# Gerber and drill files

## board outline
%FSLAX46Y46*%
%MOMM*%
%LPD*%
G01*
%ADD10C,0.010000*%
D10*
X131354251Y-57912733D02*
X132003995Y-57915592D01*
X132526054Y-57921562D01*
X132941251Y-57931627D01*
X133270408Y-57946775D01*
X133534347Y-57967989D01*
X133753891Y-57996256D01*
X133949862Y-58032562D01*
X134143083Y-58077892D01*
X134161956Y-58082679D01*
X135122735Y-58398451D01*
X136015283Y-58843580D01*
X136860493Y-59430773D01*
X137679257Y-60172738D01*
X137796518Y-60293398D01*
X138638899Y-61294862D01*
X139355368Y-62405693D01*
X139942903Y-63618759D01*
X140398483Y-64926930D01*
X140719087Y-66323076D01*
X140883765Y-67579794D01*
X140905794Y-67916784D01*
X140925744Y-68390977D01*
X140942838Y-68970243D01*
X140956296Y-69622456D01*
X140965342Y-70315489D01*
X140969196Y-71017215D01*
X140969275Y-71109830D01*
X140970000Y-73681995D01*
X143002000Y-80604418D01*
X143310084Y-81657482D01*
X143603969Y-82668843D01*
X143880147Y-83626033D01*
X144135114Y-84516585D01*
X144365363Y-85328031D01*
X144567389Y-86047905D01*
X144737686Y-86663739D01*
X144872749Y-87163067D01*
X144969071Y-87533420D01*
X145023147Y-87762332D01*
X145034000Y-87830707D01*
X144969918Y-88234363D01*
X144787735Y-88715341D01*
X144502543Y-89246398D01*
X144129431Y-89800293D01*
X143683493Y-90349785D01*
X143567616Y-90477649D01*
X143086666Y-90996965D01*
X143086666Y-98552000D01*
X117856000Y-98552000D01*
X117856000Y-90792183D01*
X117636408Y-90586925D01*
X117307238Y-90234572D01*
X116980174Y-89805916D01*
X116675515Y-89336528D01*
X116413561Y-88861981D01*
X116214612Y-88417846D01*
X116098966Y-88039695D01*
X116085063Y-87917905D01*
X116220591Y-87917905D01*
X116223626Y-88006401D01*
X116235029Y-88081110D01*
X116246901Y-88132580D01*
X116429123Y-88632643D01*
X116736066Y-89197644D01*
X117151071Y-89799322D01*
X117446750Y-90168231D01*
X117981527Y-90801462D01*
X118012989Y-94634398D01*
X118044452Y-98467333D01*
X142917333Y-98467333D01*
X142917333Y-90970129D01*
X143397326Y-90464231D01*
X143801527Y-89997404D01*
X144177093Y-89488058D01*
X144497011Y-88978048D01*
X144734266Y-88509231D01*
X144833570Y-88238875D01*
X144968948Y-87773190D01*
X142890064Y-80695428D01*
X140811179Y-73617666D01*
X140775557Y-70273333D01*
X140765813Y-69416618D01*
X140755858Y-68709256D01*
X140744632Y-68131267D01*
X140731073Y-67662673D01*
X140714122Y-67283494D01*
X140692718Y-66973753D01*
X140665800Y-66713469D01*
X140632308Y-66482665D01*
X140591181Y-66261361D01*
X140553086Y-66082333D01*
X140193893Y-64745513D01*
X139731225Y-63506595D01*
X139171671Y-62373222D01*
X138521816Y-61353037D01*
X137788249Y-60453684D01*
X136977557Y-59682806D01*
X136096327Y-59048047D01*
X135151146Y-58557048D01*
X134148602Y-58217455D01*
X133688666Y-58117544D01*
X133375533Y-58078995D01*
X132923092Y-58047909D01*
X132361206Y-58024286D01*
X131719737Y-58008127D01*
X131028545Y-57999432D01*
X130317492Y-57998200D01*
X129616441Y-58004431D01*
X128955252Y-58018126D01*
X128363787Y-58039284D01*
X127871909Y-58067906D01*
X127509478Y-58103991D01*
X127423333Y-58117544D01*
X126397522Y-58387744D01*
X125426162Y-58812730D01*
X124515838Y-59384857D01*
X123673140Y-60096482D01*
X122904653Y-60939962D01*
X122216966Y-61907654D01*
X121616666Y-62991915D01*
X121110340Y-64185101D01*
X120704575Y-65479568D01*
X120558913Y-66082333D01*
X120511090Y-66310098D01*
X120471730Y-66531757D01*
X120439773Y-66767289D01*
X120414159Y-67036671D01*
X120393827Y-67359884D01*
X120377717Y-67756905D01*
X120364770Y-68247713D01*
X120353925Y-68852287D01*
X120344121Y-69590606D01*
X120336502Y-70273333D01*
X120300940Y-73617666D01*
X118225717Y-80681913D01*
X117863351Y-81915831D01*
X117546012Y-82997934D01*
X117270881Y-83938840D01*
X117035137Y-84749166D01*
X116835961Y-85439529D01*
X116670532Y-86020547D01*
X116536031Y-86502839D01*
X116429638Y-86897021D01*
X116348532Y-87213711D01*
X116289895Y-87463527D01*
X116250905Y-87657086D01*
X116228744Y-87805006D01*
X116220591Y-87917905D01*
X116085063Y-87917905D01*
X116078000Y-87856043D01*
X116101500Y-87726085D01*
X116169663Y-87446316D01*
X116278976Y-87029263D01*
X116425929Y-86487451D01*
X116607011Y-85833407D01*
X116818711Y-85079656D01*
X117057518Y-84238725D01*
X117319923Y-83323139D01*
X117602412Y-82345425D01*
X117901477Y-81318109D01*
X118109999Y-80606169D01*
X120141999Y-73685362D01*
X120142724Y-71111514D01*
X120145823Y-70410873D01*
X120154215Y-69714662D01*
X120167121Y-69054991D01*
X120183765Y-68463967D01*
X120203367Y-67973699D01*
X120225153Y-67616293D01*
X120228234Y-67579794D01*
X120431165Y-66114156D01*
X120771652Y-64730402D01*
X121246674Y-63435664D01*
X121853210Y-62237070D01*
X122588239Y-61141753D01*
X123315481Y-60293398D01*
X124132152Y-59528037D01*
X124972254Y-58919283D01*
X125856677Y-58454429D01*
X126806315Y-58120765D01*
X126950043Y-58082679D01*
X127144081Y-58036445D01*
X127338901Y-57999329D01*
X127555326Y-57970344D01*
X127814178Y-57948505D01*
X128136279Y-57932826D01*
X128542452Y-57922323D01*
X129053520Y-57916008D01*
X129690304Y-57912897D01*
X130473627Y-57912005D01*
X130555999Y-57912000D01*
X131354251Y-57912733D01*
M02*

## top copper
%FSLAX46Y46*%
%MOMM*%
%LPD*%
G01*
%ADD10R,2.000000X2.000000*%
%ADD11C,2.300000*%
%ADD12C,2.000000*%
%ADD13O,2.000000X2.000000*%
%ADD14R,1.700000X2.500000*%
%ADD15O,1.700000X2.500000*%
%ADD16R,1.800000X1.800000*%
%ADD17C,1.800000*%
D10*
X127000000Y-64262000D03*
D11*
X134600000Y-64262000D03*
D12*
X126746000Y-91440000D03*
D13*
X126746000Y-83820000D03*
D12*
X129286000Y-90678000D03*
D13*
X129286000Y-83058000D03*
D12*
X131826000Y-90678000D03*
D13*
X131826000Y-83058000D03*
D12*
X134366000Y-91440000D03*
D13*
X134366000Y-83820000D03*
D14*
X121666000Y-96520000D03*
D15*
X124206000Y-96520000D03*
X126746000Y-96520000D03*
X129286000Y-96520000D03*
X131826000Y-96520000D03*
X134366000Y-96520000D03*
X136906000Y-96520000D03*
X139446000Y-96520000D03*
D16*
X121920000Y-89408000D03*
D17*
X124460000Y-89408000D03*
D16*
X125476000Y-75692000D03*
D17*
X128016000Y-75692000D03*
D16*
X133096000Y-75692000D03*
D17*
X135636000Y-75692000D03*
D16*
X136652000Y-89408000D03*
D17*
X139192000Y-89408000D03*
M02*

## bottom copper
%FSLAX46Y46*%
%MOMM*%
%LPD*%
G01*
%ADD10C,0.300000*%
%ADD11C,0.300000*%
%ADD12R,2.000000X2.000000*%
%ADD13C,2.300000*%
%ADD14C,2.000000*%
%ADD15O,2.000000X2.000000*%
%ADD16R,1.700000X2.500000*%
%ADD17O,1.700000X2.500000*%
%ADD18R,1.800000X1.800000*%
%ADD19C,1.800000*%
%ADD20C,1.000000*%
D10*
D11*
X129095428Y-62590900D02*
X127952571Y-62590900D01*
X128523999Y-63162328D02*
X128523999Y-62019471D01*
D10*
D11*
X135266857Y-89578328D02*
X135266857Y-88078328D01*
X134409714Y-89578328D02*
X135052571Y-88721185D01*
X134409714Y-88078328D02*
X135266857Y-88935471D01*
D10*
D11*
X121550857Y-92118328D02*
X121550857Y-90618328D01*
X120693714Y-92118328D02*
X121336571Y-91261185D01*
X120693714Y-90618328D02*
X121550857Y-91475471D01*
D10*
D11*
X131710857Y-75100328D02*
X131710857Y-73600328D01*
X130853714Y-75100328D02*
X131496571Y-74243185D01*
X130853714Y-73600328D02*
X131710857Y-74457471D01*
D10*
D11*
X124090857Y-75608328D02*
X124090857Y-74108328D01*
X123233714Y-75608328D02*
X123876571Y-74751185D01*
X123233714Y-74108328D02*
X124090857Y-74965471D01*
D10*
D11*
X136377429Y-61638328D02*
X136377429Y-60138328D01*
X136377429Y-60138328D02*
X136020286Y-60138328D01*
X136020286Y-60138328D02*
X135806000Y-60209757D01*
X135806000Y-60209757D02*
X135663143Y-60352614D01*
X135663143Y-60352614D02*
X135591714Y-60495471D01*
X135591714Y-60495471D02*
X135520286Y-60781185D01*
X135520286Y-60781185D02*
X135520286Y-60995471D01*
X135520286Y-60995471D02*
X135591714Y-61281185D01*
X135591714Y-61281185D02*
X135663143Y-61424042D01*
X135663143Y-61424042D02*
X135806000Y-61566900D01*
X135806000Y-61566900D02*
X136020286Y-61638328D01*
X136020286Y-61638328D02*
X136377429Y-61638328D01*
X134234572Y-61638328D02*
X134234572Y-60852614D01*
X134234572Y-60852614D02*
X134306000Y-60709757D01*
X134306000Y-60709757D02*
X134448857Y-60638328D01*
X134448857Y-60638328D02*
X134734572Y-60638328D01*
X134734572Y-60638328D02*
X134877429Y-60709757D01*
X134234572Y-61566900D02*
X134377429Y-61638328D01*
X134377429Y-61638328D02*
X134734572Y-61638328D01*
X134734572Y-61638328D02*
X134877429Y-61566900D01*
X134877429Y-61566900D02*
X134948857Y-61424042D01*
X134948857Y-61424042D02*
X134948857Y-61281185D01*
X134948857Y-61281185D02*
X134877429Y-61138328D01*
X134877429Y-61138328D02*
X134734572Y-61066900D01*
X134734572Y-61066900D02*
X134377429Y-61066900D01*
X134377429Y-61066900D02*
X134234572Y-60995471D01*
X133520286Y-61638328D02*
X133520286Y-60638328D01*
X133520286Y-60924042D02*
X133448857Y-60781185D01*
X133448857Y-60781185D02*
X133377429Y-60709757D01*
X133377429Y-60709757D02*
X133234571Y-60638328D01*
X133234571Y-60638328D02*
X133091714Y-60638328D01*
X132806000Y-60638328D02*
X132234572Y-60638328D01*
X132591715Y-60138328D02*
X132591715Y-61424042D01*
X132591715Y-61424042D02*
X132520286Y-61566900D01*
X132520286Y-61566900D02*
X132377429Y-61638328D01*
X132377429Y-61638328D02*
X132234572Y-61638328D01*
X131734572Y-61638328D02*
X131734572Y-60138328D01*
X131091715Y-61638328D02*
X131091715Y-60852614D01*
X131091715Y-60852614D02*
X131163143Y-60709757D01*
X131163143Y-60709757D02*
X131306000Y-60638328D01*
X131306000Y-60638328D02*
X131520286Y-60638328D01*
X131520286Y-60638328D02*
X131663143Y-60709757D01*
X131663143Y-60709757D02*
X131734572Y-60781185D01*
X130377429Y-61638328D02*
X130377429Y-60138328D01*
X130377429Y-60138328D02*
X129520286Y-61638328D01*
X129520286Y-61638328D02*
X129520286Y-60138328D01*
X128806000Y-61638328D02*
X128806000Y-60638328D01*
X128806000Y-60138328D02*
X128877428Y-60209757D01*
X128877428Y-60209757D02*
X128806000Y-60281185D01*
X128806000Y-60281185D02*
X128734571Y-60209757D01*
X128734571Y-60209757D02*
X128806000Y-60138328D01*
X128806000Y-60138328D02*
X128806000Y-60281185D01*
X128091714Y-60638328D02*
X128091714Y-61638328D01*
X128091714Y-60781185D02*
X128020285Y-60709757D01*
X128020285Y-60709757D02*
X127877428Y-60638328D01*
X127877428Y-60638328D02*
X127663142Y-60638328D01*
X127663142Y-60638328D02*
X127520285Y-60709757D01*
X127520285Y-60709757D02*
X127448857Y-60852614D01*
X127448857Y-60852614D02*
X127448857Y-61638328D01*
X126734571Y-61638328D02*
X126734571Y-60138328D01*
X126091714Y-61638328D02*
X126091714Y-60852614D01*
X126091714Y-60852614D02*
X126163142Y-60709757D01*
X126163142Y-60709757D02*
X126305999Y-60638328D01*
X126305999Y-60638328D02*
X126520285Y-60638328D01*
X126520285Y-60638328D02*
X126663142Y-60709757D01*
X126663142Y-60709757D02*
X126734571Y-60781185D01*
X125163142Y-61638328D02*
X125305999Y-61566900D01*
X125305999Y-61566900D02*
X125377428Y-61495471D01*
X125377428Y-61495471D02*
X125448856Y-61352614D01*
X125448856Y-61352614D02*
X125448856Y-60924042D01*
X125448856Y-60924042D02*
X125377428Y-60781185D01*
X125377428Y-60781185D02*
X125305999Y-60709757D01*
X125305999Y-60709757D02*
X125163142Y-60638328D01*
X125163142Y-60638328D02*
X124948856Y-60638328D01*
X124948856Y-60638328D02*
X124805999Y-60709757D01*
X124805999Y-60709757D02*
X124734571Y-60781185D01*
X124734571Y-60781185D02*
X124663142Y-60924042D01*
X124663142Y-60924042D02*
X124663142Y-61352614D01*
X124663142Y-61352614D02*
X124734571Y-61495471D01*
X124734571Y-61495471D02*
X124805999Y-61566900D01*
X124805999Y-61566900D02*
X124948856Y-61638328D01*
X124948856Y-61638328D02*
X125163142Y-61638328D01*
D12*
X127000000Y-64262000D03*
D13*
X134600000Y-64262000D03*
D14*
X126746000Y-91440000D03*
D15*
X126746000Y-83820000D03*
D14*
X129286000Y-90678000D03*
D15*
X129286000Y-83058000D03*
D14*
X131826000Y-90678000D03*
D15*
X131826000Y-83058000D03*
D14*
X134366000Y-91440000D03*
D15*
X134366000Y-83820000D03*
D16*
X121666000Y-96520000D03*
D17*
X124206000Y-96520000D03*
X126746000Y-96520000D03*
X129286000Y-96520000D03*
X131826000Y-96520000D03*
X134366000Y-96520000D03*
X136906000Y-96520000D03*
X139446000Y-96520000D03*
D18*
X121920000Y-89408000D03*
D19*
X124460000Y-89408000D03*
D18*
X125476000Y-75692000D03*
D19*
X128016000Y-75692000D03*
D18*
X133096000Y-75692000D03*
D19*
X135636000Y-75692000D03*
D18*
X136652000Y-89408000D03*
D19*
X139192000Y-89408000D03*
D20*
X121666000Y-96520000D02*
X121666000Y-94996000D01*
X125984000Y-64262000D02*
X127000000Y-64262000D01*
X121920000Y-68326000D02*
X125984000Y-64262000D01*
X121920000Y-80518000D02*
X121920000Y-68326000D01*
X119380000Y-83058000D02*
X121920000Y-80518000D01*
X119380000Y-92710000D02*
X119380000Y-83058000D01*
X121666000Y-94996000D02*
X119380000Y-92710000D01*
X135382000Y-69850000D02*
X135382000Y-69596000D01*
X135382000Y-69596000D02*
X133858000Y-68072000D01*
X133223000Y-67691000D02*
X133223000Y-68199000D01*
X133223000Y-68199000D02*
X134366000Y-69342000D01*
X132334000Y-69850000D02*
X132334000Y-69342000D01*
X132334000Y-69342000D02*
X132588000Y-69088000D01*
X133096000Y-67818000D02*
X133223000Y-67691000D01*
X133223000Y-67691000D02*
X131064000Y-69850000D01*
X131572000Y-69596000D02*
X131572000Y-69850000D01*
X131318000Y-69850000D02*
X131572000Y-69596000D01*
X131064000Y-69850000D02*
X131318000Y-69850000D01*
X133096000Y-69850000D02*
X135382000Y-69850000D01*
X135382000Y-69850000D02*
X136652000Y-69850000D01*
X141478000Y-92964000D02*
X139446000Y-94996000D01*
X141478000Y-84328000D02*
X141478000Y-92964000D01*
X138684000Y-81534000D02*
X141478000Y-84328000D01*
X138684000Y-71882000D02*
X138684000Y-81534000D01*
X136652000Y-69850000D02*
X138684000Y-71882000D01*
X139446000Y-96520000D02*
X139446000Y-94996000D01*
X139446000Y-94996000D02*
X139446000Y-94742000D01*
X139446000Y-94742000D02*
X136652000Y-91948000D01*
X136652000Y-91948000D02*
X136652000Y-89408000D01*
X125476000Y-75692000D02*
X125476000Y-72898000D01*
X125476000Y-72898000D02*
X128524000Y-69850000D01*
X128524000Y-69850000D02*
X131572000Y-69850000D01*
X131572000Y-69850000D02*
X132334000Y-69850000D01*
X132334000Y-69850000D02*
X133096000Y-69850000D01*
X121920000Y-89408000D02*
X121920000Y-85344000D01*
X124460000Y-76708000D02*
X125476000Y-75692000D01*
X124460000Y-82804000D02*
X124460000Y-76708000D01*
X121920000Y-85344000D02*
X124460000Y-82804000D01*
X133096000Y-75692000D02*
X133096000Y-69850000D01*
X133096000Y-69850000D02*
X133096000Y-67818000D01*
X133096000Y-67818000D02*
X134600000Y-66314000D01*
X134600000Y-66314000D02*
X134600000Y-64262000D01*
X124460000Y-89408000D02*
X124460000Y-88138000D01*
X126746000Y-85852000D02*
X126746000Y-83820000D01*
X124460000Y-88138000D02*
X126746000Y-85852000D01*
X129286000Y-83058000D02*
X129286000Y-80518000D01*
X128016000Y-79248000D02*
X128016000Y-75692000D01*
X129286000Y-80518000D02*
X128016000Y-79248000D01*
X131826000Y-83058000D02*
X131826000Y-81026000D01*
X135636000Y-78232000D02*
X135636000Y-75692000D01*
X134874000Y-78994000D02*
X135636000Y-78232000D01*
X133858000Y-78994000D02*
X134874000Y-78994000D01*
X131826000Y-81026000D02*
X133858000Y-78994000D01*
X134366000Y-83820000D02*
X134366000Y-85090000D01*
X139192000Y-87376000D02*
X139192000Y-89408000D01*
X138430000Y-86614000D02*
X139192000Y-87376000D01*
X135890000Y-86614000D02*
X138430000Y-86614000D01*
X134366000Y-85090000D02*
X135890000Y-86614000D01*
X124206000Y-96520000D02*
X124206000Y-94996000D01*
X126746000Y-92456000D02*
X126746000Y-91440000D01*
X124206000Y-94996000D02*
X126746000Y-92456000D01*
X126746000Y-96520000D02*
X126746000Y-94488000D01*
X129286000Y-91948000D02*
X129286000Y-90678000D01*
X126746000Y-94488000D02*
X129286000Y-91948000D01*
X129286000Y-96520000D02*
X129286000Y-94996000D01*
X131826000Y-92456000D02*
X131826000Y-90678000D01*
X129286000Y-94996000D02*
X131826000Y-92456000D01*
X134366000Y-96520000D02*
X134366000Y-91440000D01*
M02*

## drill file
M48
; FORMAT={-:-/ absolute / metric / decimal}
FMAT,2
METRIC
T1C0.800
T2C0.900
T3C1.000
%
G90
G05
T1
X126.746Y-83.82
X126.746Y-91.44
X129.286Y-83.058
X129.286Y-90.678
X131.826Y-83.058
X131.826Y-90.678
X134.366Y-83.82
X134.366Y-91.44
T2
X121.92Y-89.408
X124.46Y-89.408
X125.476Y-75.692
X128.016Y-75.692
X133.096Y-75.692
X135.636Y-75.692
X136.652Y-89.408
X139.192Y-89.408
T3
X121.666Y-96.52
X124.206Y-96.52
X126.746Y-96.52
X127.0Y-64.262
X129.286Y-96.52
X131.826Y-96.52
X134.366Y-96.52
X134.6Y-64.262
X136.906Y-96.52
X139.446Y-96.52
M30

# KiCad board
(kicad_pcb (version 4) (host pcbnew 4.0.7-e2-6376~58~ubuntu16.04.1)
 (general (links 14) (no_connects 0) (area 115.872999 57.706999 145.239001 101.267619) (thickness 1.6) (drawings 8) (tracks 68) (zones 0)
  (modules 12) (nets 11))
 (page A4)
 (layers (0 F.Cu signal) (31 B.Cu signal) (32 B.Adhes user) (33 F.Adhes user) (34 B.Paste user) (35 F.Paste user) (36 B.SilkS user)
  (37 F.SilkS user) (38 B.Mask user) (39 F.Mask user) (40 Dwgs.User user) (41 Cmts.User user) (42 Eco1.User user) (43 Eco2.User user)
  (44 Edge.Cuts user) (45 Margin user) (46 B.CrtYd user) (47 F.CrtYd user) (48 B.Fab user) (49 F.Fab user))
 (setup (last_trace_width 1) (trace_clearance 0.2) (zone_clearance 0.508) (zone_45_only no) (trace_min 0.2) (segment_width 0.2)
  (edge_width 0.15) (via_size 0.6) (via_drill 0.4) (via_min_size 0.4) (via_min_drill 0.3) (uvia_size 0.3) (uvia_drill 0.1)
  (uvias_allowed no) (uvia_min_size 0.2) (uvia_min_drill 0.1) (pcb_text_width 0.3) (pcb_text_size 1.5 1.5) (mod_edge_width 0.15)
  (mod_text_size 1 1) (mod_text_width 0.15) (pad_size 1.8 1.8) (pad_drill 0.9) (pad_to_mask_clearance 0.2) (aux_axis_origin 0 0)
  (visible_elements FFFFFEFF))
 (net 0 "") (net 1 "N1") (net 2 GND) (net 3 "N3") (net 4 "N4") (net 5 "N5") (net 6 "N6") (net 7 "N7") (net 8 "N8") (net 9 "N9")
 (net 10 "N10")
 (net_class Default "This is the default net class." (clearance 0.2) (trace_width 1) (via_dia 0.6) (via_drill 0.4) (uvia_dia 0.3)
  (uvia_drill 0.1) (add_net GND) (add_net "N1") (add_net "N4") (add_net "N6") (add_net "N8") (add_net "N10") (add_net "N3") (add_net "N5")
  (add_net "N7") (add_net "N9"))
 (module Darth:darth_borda (layer F.Cu) (at 130.556 78.232)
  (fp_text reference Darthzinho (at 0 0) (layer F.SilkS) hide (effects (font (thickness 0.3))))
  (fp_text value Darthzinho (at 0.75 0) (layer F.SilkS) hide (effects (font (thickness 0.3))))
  (fp_poly
   (pts (xy 0.798251 -20.319267) (xy 1.447995 -20.316408) (xy 1.970054 -20.310438) (xy 2.385251 -20.300373) (xy 2.714408 -20.285225)
    (xy 2.978347 -20.264011) (xy 3.197891 -20.235744) (xy 3.393862 -20.199438) (xy 3.587083 -20.154108) (xy 3.605956 -20.149321)
    (xy 4.566735 -19.833549) (xy 5.459283 -19.38842) (xy 6.304493 -18.801227) (xy 7.123257 -18.059262) (xy 7.240518 -17.938602)
    (xy 8.082899 -16.937138) (xy 8.799368 -15.826307) (xy 9.386903 -14.613241) (xy 9.842483 -13.30507) (xy 10.163087 -11.908924)
    (xy 10.327765 -10.652206) (xy 10.349794 -10.315216) (xy 10.369744 -9.841023) (xy 10.386838 -9.261757) (xy 10.400296 -8.609544)
    (xy 10.409342 -7.916511) (xy 10.413196 -7.214785) (xy 10.413275 -7.12217) (xy 10.414 -4.550005) (xy 12.446 2.372418)
    (xy 12.754084 3.425482) (xy 13.047969 4.436843) (xy 13.324147 5.394033) (xy 13.579114 6.284585) (xy 13.809363 7.096031)
    (xy 14.011389 7.815905) (xy 14.181686 8.431739) (xy 14.316749 8.931067) (xy 14.413071 9.30142) (xy 14.467147 9.530332)
    (xy 14.478 9.598707) (xy 14.413918 10.002363) (xy 14.231735 10.483341) (xy 13.946543 11.014398) (xy 13.573431 11.568293)
    (xy 13.127493 12.117785) (xy 13.011616 12.245649) (xy 12.530666 12.764965) (xy 12.530666 20.32) (xy -12.7 20.32) (xy -12.7 12.560183)
    (xy -12.919592 12.354925) (xy -13.248762 12.002572) (xy -13.575826 11.573916) (xy -13.880485 11.104528) (xy -14.142439 10.629981)
    (xy -14.341388 10.185846) (xy -14.457034 9.807695) (xy -14.470937 9.685905) (xy -14.335409 9.685905) (xy -14.332374 9.774401)
    (xy -14.320971 9.84911) (xy -14.309099 9.90058) (xy -14.126877 10.400643) (xy -13.819934 10.965644) (xy -13.404929 11.567322)
    (xy -13.10925 11.936231) (xy -12.574473 12.569462) (xy -12.543011 16.402398) (xy -12.511548 20.235333) (xy 12.361333 20.235333)
    (xy 12.361333 12.738129) (xy 12.841326 12.232231) (xy 13.245527 11.765404) (xy 13.621093 11.256058) (xy 13.941011 10.746048)
    (xy 14.178266 10.277231) (xy 14.27757 10.006875) (xy 14.412948 9.54119) (xy 12.334064 2.463428) (xy 10.255179 -4.614334)
    (xy 10.219557 -7.958667) (xy 10.209813 -8.815382) (xy 10.199858 -9.522744) (xy 10.188632 -10.100733) (xy 10.175073 -10.569327)
    (xy 10.158122 -10.948506) (xy 10.136718 -11.258247) (xy 10.1098 -11.518531) (xy 10.076308 -11.749335) (xy 10.035181 -11.970639)
    (xy 9.997086 -12.149667) (xy 9.637893 -13.486487) (xy 9.175225 -14.725405) (xy 8.615671 -15.858778) (xy 7.965816 -16.878963)
    (xy 7.232249 -17.778316) (xy 6.421557 -18.549194) (xy 5.540327 -19.183953) (xy 4.595146 -19.674952) (xy 3.592602 -20.014545)
    (xy 3.132666 -20.114456) (xy 2.819533 -20.153005) (xy 2.367092 -20.184091) (xy 1.805206 -20.207714) (xy 1.163737 -20.223873)
    (xy 0.472545 -20.232568) (xy -0.238508 -20.2338) (xy -0.939559 -20.227569) (xy -1.600748 -20.213874) (xy -2.192213 -20.192716)
    (xy -2.684091 -20.164094) (xy -3.046522 -20.128009) (xy -3.132667 -20.114456) (xy -4.158478 -19.844256) (xy -5.129838 -19.41927)
    (xy -6.040162 -18.847143) (xy -6.88286 -18.135518) (xy -7.651347 -17.292038) (xy -8.339034 -16.324346) (xy -8.939334 -15.240085)
    (xy -9.44566 -14.046899) (xy -9.851425 -12.752432) (xy -9.997087 -12.149667) (xy -10.04491 -11.921902) (xy -10.08427 -11.700243)
    (xy -10.116227 -11.464711) (xy -10.141841 -11.195329) (xy -10.162173 -10.872116) (xy -10.178283 -10.475095) (xy -10.19123 -9.984287)
    (xy -10.202075 -9.379713) (xy -10.211879 -8.641394) (xy -10.219498 -7.958667) (xy -10.25506 -4.614334) (xy -12.330283 2.449913)
    (xy -12.692649 3.683831) (xy -13.009988 4.765934) (xy -13.285119 5.70684) (xy -13.520863 6.517166) (xy -13.720039 7.207529)
    (xy -13.885468 7.788547) (xy -14.019969 8.270839) (xy -14.126362 8.665021) (xy -14.207468 8.981711) (xy -14.266105 9.231527)
    (xy -14.305095 9.425086) (xy -14.327256 9.573006) (xy -14.335409 9.685905) (xy -14.470937 9.685905) (xy -14.478 9.624043)
    (xy -14.4545 9.494085) (xy -14.386337 9.214316) (xy -14.277024 8.797263) (xy -14.130071 8.255451) (xy -13.948989 7.601407)
    (xy -13.737289 6.847656) (xy -13.498482 6.006725) (xy -13.236077 5.091139) (xy -12.953588 4.113425) (xy -12.654523 3.086109)
    (xy -12.446001 2.374169) (xy -10.414001 -4.546638) (xy -10.413276 -7.120486) (xy -10.410177 -7.821127) (xy -10.401785 -8.517338)
    (xy -10.388879 -9.177009) (xy -10.372235 -9.768033) (xy -10.352633 -10.258301) (xy -10.330847 -10.615707) (xy -10.327766 -10.652206)
    (xy -10.124835 -12.117844) (xy -9.784348 -13.501598) (xy -9.309326 -14.796336) (xy -8.70279 -15.99493) (xy -7.967761 -17.090247)
    (xy -7.240519 -17.938602) (xy -6.423848 -18.703963) (xy -5.583746 -19.312717) (xy -4.699323 -19.777571) (xy -3.749685 -20.111235)
    (xy -3.605957 -20.149321) (xy -3.411919 -20.195555) (xy -3.217099 -20.232671) (xy -3.000674 -20.261656) (xy -2.741822 -20.283495)
    (xy -2.419721 -20.299174) (xy -2.013548 -20.309677) (xy -1.50248 -20.315992) (xy -0.865696 -20.319103) (xy -0.082373 -20.319995)
    (xy -0.000001 -20.32) (xy 0.798251 -20.319267))
   (layer Edge.Cuts) (width 0.01)))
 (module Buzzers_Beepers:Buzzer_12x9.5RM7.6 (layer F.Cu) (at 127 64.262)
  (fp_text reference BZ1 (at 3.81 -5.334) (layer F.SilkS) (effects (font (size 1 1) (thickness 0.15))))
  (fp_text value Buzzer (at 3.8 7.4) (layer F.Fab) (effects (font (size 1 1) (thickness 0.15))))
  (pad 1 thru_hole rect (at 0 0) (size 2 2) (drill 1) (layers *.Cu *.Mask) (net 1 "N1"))
  (pad 2 thru_hole circle (at 7.6 0) (size 2.3 2.3) (drill 1) (layers *.Cu *.Mask) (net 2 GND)))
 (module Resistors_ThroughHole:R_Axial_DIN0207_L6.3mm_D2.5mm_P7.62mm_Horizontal (layer F.Cu) (at 126.746 91.44 90)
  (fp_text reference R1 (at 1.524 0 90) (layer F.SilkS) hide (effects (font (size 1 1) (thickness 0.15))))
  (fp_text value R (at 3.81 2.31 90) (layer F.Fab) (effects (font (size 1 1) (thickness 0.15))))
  (pad 1 thru_hole circle (at 0 0 90) (size 2 2) (drill 0.8) (layers *.Cu *.Mask) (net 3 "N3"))
  (pad 2 thru_hole oval (at 7.62 0 90) (size 2 2) (drill 0.8) (layers *.Cu *.Mask) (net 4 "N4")))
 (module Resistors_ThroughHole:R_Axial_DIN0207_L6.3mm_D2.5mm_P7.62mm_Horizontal (layer F.Cu) (at 129.286 90.678 90)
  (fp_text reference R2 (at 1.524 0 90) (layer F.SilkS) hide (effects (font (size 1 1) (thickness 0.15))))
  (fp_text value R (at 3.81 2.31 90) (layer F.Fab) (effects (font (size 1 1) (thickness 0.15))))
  (pad 1 thru_hole circle (at 0 0 90) (size 2 2) (drill 0.8) (layers *.Cu *.Mask) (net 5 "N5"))
  (pad 2 thru_hole oval (at 7.62 0 90) (size 2 2) (drill 0.8) (layers *.Cu *.Mask) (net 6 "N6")))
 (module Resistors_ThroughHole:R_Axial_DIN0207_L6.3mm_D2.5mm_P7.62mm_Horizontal (layer F.Cu) (at 131.826 90.678 90)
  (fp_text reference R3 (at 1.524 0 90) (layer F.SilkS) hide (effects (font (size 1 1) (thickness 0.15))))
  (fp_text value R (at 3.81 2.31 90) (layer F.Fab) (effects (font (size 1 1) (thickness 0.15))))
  (pad 1 thru_hole circle (at 0 0 90) (size 2 2) (drill 0.8) (layers *.Cu *.Mask) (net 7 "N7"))
  (pad 2 thru_hole oval (at 7.62 0 90) (size 2 2) (drill 0.8) (layers *.Cu *.Mask) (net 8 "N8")))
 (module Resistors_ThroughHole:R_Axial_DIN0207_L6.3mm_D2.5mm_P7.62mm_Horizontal (layer F.Cu) (at 134.366 91.44 90)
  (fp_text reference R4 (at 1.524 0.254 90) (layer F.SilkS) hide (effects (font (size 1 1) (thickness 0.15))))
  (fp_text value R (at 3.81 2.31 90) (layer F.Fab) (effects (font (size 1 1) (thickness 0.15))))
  (pad 1 thru_hole circle (at 0 0 90) (size 2 2) (drill 0.8) (layers *.Cu *.Mask) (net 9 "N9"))
  (pad 2 thru_hole oval (at 7.62 0 90) (size 2 2) (drill 0.8) (layers *.Cu *.Mask) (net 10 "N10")))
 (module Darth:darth (layer F.Cu) (at 130.556 76.454)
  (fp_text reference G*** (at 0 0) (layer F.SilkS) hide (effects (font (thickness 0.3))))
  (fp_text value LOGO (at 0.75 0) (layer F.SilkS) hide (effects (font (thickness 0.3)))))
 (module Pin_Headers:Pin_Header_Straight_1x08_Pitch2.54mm (layer F.Cu) (at 121.666 96.52 90)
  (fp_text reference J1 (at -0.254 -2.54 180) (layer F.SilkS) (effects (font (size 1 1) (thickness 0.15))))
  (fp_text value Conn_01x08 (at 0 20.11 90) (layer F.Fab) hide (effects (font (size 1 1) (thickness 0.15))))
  (pad 1 thru_hole rect (at 0 0 90) (size 2.5 1.7) (drill 1) (layers *.Cu *.Mask) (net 1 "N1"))
  (pad 2 thru_hole oval (at 0 2.54 90) (size 2.5 1.7) (drill 1) (layers *.Cu *.Mask) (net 3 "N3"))
  (pad 3 thru_hole oval (at 0 5.08 90) (size 2.5 1.7) (drill 1) (layers *.Cu *.Mask) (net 5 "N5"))
  (pad 4 thru_hole oval (at 0 7.62 90) (size 2.5 1.7) (drill 1) (layers *.Cu *.Mask) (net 7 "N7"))
  (pad 5 thru_hole oval (at 0 10.16 90) (size 2.5 1.7) (drill 1) (layers *.Cu *.Mask))
  (pad 6 thru_hole oval (at 0 12.7 90) (size 2.5 1.7) (drill 1) (layers *.Cu *.Mask) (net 9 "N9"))
  (pad 7 thru_hole oval (at 0 15.24 90) (size 2.5 1.7) (drill 1) (layers *.Cu *.Mask))
  (pad 8 thru_hole oval (at 0 17.78 90) (size 2.5 1.7) (drill 1) (layers *.Cu *.Mask) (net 2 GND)))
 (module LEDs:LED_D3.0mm (layer F.Cu) (at 121.92 89.408)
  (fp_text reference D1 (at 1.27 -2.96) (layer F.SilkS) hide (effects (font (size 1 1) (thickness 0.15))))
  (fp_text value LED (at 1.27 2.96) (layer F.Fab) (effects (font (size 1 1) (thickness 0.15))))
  (pad 1 thru_hole rect (at 0 0) (size 1.8 1.8) (drill 0.9) (layers *.Cu *.Mask) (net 2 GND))
  (pad 2 thru_hole circle (at 2.54 0) (size 1.8 1.8) (drill 0.9) (layers *.Cu *.Mask) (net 4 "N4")))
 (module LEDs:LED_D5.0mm (layer F.Cu) (at 125.476 75.692)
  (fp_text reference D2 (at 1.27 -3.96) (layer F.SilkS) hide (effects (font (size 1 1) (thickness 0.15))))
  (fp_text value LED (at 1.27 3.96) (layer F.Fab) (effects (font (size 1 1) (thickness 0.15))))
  (pad 1 thru_hole rect (at 0 0) (size 1.8 1.8) (drill 0.9) (layers *.Cu *.Mask) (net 2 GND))
  (pad 2 thru_hole circle (at 2.54 0) (size 1.8 1.8) (drill 0.9) (layers *.Cu *.Mask) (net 6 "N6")))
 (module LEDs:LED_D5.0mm (layer F.Cu) (at 133.096 75.692)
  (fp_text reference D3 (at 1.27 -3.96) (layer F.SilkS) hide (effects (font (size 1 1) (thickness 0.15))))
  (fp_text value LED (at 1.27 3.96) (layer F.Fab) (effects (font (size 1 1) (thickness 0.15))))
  (pad 1 thru_hole rect (at 0 0) (size 1.8 1.8) (drill 0.9) (layers *.Cu *.Mask) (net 2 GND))
  (pad 2 thru_hole circle (at 2.54 0) (size 1.8 1.8) (drill 0.9) (layers *.Cu *.Mask) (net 8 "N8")))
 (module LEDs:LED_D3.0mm (layer F.Cu) (at 136.652 89.408)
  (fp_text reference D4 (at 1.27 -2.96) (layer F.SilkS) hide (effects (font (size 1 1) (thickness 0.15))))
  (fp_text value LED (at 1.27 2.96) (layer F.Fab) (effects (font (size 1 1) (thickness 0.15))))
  (pad 1 thru_hole rect (at 0 0) (size 1.8 1.8) (drill 0.9) (layers *.Cu *.Mask) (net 2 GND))
  (pad 2 thru_hole circle (at 2.54 0) (size 1.8 1.8) (drill 0.9) (layers *.Cu *.Mask) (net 10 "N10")))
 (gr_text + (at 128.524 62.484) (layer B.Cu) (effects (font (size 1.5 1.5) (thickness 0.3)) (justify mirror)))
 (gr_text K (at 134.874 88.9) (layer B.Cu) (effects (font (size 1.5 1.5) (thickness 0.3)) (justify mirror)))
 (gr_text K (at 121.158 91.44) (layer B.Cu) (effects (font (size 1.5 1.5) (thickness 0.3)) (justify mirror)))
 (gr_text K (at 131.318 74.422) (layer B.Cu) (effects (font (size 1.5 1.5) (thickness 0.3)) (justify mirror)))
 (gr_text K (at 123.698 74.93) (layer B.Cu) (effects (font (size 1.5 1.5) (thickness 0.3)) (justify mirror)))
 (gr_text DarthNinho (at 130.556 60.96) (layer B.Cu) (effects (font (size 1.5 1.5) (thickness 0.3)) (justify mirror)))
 (segment (start 121.666 96.52) (end 121.666 94.996) (width 1) (layer B.Cu) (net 1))
 (segment (start 125.984 64.262) (end 127 64.262) (width 1) (layer B.Cu) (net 1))
 (segment (start 121.92 68.326) (end 125.984 64.262) (width 1) (layer B.Cu) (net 1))
 (segment (start 121.92 80.518) (end 121.92 68.326) (width 1) (layer B.Cu) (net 1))
 (segment (start 119.38 83.058) (end 121.92 80.518) (width 1) (layer B.Cu) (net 1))
 (segment (start 119.38 92.71) (end 119.38 83.058) (width 1) (layer B.Cu) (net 1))
 (segment (start 121.666 94.996) (end 119.38 92.71) (width 1) (layer B.Cu) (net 1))
 (segment (start 135.382 69.85) (end 135.382 69.596) (width 1) (layer B.Cu) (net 2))
 (segment (start 135.382 69.596) (end 133.858 68.072) (width 1) (layer B.Cu) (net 2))
 (segment (start 133.223 67.691) (end 133.223 68.199) (width 1) (layer B.Cu) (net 2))
 (segment (start 133.223 68.199) (end 134.366 69.342) (width 1) (layer B.Cu) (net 2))
 (segment (start 132.334 69.85) (end 132.334 69.342) (width 1) (layer B.Cu) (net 2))
 (segment (start 132.334 69.342) (end 132.588 69.088) (width 1) (layer B.Cu) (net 2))
 (segment (start 133.096 67.818) (end 133.223 67.691) (width 1) (layer B.Cu) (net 2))
 (segment (start 133.223 67.691) (end 131.064 69.85) (width 1) (layer B.Cu) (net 2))
 (segment (start 131.572 69.596) (end 131.572 69.85) (width 1) (layer B.Cu) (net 2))
 (segment (start 131.318 69.85) (end 131.572 69.596) (width 1) (layer B.Cu) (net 2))
 (segment (start 131.064 69.85) (end 131.318 69.85) (width 1) (layer B.Cu) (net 2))
 (segment (start 133.096 69.85) (end 135.382 69.85) (width 1) (layer B.Cu) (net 2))
 (segment (start 135.382 69.85) (end 136.652 69.85) (width 1) (layer B.Cu) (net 2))
 (segment (start 141.478 92.964) (end 139.446 94.996) (width 1) (layer B.Cu) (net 2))
 (segment (start 141.478 84.328) (end 141.478 92.964) (width 1) (layer B.Cu) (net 2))
 (segment (start 138.684 81.534) (end 141.478 84.328) (width 1) (layer B.Cu) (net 2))
 (segment (start 138.684 71.882) (end 138.684 81.534) (width 1) (layer B.Cu) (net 2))
 (segment (start 136.652 69.85) (end 138.684 71.882) (width 1) (layer B.Cu) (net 2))
 (segment (start 139.446 96.52) (end 139.446 94.996) (width 1) (layer B.Cu) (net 2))
 (segment (start 139.446 94.996) (end 139.446 94.742) (width 1) (layer B.Cu) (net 2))
 (segment (start 139.446 94.742) (end 136.652 91.948) (width 1) (layer B.Cu) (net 2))
 (segment (start 136.652 91.948) (end 136.652 89.408) (width 1) (layer B.Cu) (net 2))
 (segment (start 125.476 75.692) (end 125.476 72.898) (width 1) (layer B.Cu) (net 2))
 (segment (start 125.476 72.898) (end 128.524 69.85) (width 1) (layer B.Cu) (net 2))
 (segment (start 128.524 69.85) (end 131.572 69.85) (width 1) (layer B.Cu) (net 2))
 (segment (start 131.572 69.85) (end 132.334 69.85) (width 1) (layer B.Cu) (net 2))
 (segment (start 132.334 69.85) (end 133.096 69.85) (width 1) (layer B.Cu) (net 2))
 (segment (start 121.92 89.408) (end 121.92 85.344) (width 1) (layer B.Cu) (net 2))
 (segment (start 124.46 76.708) (end 125.476 75.692) (width 1) (layer B.Cu) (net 2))
 (segment (start 124.46 82.804) (end 124.46 76.708) (width 1) (layer B.Cu) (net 2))
 (segment (start 121.92 85.344) (end 124.46 82.804) (width 1) (layer B.Cu) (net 2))
 (segment (start 133.096 75.692) (end 133.096 69.85) (width 1) (layer B.Cu) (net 2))
 (segment (start 133.096 69.85) (end 133.096 67.818) (width 1) (layer B.Cu) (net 2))
 (segment (start 133.096 67.818) (end 134.6 66.314) (width 1) (layer B.Cu) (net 2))
 (segment (start 134.6 66.314) (end 134.6 64.262) (width 1) (layer B.Cu) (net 2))
 (segment (start 124.46 89.408) (end 124.46 88.138) (width 1) (layer B.Cu) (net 4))
 (segment (start 126.746 85.852) (end 126.746 83.82) (width 1) (layer B.Cu) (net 4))
 (segment (start 124.46 88.138) (end 126.746 85.852) (width 1) (layer B.Cu) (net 4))
 (segment (start 129.286 83.058) (end 129.286 80.518) (width 1) (layer B.Cu) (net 6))
 (segment (start 128.016 79.248) (end 128.016 75.692) (width 1) (layer B.Cu) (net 6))
 (segment (start 129.286 80.518) (end 128.016 79.248) (width 1) (layer B.Cu) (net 6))
 (segment (start 131.826 83.058) (end 131.826 81.026) (width 1) (layer B.Cu) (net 8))
 (segment (start 135.636 78.232) (end 135.636 75.692) (width 1) (layer B.Cu) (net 8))
 (segment (start 134.874 78.994) (end 135.636 78.232) (width 1) (layer B.Cu) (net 8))
 (segment (start 133.858 78.994) (end 134.874 78.994) (width 1) (layer B.Cu) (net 8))
 (segment (start 131.826 81.026) (end 133.858 78.994) (width 1) (layer B.Cu) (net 8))
 (segment (start 134.366 83.82) (end 134.366 85.09) (width 1) (layer B.Cu) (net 10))
 (segment (start 139.192 87.376) (end 139.192 89.408) (width 1) (layer B.Cu) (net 10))
 (segment (start 138.43 86.614) (end 139.192 87.376) (width 1) (layer B.Cu) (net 10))
 (segment (start 135.89 86.614) (end 138.43 86.614) (width 1) (layer B.Cu) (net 10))
 (segment (start 134.366 85.09) (end 135.89 86.614) (width 1) (layer B.Cu) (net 10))
 (segment (start 124.206 96.52) (end 124.206 94.996) (width 1) (layer B.Cu) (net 3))
 (segment (start 126.746 92.456) (end 126.746 91.44) (width 1) (layer B.Cu) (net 3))
 (segment (start 124.206 94.996) (end 126.746 92.456) (width 1) (layer B.Cu) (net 3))
 (segment (start 126.746 96.52) (end 126.746 94.488) (width 1) (layer B.Cu) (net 5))
 (segment (start 129.286 91.948) (end 129.286 90.678) (width 1) (layer B.Cu) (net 5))
 (segment (start 126.746 94.488) (end 129.286 91.948) (width 1) (layer B.Cu) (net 5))
 (segment (start 129.286 96.52) (end 129.286 94.996) (width 1) (layer B.Cu) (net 7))
 (segment (start 131.826 92.456) (end 131.826 90.678) (width 1) (layer B.Cu) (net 7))
 (segment (start 129.286 94.996) (end 131.826 92.456) (width 1) (layer B.Cu) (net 7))
 (segment (start 134.366 96.52) (end 134.366 91.44) (width 1) (layer B.Cu) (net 9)))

